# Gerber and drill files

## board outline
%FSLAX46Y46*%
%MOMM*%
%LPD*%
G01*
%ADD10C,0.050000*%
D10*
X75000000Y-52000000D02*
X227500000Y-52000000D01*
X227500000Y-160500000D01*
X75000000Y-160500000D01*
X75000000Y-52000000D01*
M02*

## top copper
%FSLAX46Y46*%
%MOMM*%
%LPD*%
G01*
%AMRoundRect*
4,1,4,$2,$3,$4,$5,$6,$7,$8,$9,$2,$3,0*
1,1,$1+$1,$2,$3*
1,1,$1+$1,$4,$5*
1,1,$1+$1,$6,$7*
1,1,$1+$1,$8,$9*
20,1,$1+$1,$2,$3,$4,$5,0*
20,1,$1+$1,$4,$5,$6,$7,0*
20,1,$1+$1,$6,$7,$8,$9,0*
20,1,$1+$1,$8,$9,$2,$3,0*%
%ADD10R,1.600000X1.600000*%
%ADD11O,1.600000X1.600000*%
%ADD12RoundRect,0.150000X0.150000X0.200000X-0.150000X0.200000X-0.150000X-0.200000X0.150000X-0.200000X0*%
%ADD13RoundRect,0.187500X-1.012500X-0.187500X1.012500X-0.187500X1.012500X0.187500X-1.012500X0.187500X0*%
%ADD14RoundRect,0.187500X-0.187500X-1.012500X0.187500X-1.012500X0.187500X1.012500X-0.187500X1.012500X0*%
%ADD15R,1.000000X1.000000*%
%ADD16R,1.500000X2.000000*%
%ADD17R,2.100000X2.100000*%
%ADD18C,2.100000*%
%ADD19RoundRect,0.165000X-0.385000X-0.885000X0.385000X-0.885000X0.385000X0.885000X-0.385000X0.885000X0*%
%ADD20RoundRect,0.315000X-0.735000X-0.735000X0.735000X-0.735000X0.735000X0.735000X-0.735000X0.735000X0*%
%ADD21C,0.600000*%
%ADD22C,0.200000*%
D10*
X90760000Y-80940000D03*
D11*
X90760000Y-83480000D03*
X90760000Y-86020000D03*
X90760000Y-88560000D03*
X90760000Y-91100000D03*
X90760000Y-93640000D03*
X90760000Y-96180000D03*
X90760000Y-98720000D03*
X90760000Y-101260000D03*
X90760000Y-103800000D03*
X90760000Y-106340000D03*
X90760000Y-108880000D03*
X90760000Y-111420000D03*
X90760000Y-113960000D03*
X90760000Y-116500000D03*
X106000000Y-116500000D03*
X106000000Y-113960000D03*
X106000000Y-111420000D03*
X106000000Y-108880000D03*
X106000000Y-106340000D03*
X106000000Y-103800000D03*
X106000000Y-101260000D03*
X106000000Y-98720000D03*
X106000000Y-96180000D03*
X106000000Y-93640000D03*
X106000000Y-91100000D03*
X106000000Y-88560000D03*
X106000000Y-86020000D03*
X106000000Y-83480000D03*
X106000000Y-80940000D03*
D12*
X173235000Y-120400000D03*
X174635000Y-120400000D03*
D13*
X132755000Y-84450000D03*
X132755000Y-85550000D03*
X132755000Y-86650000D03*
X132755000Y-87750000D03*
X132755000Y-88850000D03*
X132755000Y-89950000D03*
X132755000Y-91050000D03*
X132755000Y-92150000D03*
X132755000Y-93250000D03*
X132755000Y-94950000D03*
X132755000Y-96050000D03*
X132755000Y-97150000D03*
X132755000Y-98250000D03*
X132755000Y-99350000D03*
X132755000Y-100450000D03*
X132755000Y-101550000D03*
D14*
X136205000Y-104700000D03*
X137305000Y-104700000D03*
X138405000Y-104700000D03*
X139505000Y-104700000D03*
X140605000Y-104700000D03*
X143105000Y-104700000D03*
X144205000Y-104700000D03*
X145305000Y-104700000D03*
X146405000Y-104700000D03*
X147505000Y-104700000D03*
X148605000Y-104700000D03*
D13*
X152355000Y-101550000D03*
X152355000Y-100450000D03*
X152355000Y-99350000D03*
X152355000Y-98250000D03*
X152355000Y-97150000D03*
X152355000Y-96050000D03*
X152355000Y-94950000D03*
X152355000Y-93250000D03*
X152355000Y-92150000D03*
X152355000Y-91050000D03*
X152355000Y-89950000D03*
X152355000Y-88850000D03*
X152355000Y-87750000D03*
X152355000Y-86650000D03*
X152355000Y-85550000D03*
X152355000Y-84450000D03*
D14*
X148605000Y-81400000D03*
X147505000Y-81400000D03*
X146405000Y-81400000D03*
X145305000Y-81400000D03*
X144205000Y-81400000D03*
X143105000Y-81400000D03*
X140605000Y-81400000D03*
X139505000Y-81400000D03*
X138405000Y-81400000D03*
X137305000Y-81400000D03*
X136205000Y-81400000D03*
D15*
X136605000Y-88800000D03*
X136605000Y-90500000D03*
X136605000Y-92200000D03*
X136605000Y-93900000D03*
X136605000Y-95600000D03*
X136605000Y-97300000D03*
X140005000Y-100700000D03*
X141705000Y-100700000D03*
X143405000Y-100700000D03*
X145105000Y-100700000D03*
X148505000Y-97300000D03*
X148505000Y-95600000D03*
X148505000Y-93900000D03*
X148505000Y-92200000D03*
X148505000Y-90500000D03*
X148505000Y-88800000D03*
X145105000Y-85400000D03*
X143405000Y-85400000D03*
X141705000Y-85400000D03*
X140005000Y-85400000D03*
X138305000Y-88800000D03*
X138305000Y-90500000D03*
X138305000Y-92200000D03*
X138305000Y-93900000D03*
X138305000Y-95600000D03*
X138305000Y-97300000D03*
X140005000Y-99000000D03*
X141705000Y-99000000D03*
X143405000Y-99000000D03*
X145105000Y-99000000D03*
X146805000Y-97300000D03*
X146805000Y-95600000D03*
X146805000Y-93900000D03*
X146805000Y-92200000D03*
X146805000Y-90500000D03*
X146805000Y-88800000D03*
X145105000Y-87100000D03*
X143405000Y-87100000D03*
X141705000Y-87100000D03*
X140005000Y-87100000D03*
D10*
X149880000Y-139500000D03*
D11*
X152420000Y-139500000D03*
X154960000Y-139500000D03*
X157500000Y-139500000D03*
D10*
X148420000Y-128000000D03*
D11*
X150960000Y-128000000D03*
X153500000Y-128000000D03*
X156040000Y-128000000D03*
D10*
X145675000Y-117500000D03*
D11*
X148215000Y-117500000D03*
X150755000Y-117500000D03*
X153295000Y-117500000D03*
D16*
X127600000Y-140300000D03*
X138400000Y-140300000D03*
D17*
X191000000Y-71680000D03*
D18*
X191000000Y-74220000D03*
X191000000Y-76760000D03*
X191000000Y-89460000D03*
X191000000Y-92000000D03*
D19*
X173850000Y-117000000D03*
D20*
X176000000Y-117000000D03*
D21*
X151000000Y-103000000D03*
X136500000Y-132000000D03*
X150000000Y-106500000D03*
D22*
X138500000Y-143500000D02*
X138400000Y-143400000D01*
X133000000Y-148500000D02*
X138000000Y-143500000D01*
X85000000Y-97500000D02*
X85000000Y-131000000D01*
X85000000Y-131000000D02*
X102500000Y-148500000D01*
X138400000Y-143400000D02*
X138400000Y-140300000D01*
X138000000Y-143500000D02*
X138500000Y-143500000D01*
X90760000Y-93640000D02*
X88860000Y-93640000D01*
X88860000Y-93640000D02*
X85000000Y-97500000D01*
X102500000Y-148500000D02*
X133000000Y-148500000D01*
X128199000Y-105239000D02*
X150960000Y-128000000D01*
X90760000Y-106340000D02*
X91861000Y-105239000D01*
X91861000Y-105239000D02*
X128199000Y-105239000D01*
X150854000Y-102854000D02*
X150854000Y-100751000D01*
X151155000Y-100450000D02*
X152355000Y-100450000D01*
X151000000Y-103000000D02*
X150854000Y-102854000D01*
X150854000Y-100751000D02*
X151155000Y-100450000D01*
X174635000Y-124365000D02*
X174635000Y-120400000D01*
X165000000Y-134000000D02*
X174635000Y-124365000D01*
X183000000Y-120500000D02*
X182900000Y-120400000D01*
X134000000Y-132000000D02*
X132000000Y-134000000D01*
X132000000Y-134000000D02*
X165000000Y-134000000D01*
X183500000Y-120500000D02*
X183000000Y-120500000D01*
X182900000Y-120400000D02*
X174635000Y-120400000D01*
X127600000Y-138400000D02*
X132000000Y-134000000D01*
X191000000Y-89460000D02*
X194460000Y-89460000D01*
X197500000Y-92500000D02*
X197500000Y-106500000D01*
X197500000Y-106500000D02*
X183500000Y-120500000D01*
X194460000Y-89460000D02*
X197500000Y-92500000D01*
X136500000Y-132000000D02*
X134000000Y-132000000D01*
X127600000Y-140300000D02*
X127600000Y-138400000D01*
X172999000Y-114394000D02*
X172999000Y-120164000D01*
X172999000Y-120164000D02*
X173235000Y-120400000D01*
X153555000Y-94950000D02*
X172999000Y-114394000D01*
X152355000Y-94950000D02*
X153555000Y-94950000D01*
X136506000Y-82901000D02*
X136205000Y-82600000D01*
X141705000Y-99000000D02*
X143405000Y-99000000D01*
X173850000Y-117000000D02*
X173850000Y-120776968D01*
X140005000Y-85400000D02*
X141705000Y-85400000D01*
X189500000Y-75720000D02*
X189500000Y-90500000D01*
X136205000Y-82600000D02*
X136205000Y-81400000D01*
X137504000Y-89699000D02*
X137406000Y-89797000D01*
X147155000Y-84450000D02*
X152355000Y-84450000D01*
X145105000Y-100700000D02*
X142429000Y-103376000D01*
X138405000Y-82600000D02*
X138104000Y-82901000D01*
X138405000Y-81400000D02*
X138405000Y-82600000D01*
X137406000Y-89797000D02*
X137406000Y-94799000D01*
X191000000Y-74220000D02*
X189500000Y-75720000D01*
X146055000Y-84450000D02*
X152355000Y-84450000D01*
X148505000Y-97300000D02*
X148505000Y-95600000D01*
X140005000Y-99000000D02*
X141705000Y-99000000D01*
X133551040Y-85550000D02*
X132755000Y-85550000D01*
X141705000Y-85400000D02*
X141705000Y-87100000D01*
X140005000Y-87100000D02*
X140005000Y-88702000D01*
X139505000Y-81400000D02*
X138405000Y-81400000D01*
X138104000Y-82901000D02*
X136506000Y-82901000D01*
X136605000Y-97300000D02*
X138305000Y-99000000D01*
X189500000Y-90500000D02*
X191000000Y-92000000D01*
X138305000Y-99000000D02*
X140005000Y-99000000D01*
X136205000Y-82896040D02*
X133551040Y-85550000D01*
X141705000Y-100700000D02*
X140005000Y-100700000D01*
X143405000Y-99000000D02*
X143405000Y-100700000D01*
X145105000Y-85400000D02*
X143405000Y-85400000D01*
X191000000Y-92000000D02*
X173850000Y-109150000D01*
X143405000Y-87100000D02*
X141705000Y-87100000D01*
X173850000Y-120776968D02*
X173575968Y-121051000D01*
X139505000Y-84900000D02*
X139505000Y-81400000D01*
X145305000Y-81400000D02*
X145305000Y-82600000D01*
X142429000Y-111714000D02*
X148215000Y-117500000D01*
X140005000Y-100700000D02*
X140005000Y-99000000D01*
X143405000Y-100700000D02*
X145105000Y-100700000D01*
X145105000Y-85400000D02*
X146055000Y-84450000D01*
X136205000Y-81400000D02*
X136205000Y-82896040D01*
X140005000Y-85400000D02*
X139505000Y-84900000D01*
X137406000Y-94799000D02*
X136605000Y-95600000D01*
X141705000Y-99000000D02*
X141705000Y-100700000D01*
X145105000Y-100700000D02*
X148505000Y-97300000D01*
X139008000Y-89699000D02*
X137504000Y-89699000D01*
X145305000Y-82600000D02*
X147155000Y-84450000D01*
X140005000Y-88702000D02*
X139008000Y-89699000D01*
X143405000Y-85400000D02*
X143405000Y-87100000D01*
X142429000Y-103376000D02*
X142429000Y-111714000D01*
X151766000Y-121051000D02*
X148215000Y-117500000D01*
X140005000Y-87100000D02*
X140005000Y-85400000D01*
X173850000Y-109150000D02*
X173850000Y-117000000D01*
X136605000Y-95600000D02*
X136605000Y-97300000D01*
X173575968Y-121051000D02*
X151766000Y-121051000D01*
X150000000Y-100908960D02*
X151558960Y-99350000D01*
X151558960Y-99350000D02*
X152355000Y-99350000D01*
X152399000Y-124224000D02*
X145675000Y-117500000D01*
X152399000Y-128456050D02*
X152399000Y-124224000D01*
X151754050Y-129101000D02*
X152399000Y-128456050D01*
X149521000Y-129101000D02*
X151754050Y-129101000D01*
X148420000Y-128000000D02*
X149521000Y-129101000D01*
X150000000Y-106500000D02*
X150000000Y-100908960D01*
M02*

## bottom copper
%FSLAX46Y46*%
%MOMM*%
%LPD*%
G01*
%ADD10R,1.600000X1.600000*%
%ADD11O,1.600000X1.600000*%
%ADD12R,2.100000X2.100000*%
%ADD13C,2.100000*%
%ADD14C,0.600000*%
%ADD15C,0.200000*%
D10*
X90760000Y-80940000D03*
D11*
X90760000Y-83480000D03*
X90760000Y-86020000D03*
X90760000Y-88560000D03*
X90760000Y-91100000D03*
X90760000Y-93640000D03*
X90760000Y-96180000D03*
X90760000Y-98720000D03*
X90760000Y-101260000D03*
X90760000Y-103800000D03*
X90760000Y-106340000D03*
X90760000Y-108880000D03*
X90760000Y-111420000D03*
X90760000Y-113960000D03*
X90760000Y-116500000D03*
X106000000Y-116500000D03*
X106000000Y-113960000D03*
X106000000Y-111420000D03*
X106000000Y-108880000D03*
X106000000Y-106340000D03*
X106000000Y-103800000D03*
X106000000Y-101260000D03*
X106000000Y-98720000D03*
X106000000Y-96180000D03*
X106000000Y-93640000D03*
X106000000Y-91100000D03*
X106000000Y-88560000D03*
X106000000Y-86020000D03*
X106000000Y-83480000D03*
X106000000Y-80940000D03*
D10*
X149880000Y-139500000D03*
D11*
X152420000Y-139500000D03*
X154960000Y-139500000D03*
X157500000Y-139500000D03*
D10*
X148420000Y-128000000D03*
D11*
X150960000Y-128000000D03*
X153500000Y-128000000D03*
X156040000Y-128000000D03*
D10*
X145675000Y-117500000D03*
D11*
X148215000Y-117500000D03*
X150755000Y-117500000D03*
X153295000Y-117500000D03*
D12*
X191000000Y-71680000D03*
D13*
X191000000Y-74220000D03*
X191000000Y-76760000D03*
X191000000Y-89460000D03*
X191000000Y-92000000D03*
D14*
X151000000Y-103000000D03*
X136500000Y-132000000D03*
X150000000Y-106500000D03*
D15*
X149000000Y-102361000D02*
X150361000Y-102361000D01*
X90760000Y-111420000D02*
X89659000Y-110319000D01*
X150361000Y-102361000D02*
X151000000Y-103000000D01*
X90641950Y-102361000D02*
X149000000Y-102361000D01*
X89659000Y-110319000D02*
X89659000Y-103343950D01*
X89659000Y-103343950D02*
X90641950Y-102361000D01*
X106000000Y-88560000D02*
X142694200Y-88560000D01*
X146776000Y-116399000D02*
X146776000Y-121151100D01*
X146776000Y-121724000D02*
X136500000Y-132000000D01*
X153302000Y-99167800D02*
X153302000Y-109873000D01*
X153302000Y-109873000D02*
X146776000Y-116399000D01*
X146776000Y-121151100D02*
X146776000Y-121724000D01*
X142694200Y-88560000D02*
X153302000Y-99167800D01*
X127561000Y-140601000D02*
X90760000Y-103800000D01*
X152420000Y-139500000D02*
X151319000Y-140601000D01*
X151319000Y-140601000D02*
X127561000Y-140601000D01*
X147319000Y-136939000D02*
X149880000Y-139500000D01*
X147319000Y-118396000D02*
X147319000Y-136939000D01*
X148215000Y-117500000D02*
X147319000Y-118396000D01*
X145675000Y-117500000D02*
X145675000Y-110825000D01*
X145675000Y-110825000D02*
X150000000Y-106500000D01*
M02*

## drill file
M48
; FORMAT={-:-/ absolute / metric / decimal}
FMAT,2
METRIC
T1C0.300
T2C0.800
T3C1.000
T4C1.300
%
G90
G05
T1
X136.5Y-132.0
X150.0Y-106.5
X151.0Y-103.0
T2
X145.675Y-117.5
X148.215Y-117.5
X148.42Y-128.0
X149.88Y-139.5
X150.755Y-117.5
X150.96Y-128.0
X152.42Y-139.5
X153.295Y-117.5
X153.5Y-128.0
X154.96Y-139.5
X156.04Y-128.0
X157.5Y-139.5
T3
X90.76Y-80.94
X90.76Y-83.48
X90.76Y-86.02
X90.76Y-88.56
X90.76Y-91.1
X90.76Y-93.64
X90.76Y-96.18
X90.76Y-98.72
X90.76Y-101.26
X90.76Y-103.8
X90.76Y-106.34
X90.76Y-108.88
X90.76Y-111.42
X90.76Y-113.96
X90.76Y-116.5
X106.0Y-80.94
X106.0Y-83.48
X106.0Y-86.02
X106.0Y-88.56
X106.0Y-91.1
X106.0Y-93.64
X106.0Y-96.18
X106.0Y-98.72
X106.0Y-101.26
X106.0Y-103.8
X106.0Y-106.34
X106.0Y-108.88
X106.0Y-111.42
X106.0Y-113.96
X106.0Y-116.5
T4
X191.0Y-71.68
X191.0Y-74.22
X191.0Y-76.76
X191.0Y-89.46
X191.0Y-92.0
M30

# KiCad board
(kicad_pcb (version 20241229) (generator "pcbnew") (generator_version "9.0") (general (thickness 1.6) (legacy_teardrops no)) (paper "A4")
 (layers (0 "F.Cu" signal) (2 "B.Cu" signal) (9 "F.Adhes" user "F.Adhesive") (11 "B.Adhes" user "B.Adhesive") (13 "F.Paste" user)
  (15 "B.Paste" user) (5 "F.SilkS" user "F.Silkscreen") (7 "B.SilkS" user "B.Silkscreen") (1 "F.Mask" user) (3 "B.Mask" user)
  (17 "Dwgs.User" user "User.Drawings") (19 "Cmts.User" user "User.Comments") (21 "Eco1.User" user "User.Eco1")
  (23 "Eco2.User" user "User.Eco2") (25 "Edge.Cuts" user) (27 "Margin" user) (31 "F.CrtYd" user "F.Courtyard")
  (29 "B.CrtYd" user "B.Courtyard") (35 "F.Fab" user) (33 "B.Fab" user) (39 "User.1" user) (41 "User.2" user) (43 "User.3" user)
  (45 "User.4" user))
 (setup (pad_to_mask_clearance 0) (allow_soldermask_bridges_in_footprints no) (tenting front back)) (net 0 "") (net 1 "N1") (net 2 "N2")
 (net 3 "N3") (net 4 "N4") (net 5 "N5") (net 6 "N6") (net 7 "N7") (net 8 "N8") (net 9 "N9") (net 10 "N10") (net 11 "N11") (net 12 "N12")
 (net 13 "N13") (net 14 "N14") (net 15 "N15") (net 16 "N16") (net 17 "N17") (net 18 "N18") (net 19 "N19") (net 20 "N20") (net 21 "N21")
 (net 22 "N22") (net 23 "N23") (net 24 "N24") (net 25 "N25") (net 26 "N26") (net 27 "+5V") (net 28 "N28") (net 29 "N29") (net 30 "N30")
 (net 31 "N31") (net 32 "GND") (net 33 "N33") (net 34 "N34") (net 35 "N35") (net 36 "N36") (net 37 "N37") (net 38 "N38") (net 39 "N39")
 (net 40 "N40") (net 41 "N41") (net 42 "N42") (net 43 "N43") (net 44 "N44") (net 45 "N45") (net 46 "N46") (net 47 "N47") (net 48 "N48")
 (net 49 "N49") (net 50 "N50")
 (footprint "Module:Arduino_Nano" (layer "F.Cu") (at 90.76 80.94)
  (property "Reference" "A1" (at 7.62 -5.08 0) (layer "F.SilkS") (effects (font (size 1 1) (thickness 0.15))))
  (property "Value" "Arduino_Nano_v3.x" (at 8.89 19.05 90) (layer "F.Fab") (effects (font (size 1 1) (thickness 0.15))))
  (pad "1" thru_hole rect (at 0 0) (size 1.6 1.6) (drill 1) (layers "*.Cu" "*.Mask") (remove_unused_layers no) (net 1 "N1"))
  (pad "2" thru_hole oval (at 0 2.54) (size 1.6 1.6) (drill 1) (layers "*.Cu" "*.Mask") (remove_unused_layers no) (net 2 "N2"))
  (pad "3" thru_hole oval (at 0 5.08) (size 1.6 1.6) (drill 1) (layers "*.Cu" "*.Mask") (remove_unused_layers no) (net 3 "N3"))
  (pad "4" thru_hole oval (at 0 7.62) (size 1.6 1.6) (drill 1) (layers "*.Cu" "*.Mask") (remove_unused_layers no) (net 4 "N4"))
  (pad "5" thru_hole oval (at 0 10.16) (size 1.6 1.6) (drill 1) (layers "*.Cu" "*.Mask") (remove_unused_layers no) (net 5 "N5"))
  (pad "6" thru_hole oval (at 0 12.7) (size 1.6 1.6) (drill 1) (layers "*.Cu" "*.Mask") (remove_unused_layers no) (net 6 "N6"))
  (pad "7" thru_hole oval (at 0 15.24) (size 1.6 1.6) (drill 1) (layers "*.Cu" "*.Mask") (remove_unused_layers no) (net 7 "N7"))
  (pad "8" thru_hole oval (at 0 17.78) (size 1.6 1.6) (drill 1) (layers "*.Cu" "*.Mask") (remove_unused_layers no) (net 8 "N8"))
  (pad "9" thru_hole oval (at 0 20.32) (size 1.6 1.6) (drill 1) (layers "*.Cu" "*.Mask") (remove_unused_layers no) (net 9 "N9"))
  (pad "10" thru_hole oval (at 0 22.86) (size 1.6 1.6) (drill 1) (layers "*.Cu" "*.Mask") (remove_unused_layers no) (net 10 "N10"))
  (pad "11" thru_hole oval (at 0 25.4) (size 1.6 1.6) (drill 1) (layers "*.Cu" "*.Mask") (remove_unused_layers no) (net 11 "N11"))
  (pad "12" thru_hole oval (at 0 27.94) (size 1.6 1.6) (drill 1) (layers "*.Cu" "*.Mask") (remove_unused_layers no) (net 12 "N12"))
  (pad "13" thru_hole oval (at 0 30.48) (size 1.6 1.6) (drill 1) (layers "*.Cu" "*.Mask") (remove_unused_layers no) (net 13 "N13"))
  (pad "14" thru_hole oval (at 0 33.02) (size 1.6 1.6) (drill 1) (layers "*.Cu" "*.Mask") (remove_unused_layers no) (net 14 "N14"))
  (pad "15" thru_hole oval (at 0 35.56) (size 1.6 1.6) (drill 1) (layers "*.Cu" "*.Mask") (remove_unused_layers no) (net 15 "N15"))
  (pad "16" thru_hole oval (at 15.24 35.56) (size 1.6 1.6) (drill 1) (layers "*.Cu" "*.Mask") (remove_unused_layers no) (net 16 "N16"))
  (pad "17" thru_hole oval (at 15.24 33.02) (size 1.6 1.6) (drill 1) (layers "*.Cu" "*.Mask") (remove_unused_layers no) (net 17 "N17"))
  (pad "18" thru_hole oval (at 15.24 30.48) (size 1.6 1.6) (drill 1) (layers "*.Cu" "*.Mask") (remove_unused_layers no) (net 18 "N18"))
  (pad "19" thru_hole oval (at 15.24 27.94) (size 1.6 1.6) (drill 1) (layers "*.Cu" "*.Mask") (remove_unused_layers no) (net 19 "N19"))
  (pad "20" thru_hole oval (at 15.24 25.4) (size 1.6 1.6) (drill 1) (layers "*.Cu" "*.Mask") (remove_unused_layers no) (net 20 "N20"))
  (pad "21" thru_hole oval (at 15.24 22.86) (size 1.6 1.6) (drill 1) (layers "*.Cu" "*.Mask") (remove_unused_layers no) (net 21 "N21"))
  (pad "22" thru_hole oval (at 15.24 20.32) (size 1.6 1.6) (drill 1) (layers "*.Cu" "*.Mask") (remove_unused_layers no) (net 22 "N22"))
  (pad "23" thru_hole oval (at 15.24 17.78) (size 1.6 1.6) (drill 1) (layers "*.Cu" "*.Mask") (remove_unused_layers no) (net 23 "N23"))
  (pad "24" thru_hole oval (at 15.24 15.24) (size 1.6 1.6) (drill 1) (layers "*.Cu" "*.Mask") (remove_unused_layers no) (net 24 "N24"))
  (pad "25" thru_hole oval (at 15.24 12.7) (size 1.6 1.6) (drill 1) (layers "*.Cu" "*.Mask") (remove_unused_layers no) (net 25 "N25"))
  (pad "26" thru_hole oval (at 15.24 10.16) (size 1.6 1.6) (drill 1) (layers "*.Cu" "*.Mask") (remove_unused_layers no) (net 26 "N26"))
  (pad "27" thru_hole oval (at 15.24 7.62) (size 1.6 1.6) (drill 1) (layers "*.Cu" "*.Mask") (remove_unused_layers no) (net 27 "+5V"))
  (pad "28" thru_hole oval (at 15.24 5.08) (size 1.6 1.6) (drill 1) (layers "*.Cu" "*.Mask") (remove_unused_layers no) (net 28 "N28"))
  (pad "29" thru_hole oval (at 15.24 2.54) (size 1.6 1.6) (drill 1) (layers "*.Cu" "*.Mask") (remove_unused_layers no) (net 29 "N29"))
  (pad "30" thru_hole oval (at 15.24 0) (size 1.6 1.6) (drill 1) (layers "*.Cu" "*.Mask") (remove_unused_layers no) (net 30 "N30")))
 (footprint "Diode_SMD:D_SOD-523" (layer "F.Cu") (at 173.935 120.4)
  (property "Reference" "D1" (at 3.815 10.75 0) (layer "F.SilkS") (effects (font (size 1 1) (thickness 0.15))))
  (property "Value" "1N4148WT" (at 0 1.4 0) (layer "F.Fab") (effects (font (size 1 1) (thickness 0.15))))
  (pad "1" smd roundrect (at -0.7 0 180) (size 0.6 0.7) (layers "F.Cu" "F.Mask" "F.Paste") (roundrect_rratio 0.25) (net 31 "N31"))
  (pad "2" smd roundrect (at 0.7 0 180) (size 0.6 0.7) (layers "F.Cu" "F.Mask" "F.Paste") (roundrect_rratio 0.25) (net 27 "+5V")))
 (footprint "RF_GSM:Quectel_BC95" (layer "F.Cu") (at 142.555 93.05)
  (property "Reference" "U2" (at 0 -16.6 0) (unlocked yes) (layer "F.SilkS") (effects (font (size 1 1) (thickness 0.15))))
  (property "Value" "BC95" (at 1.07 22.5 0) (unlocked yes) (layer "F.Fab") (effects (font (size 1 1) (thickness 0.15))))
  (pad "" smd roundrect (at -10.1 -8.6) (size 2.6 0.6375) (layers "F.Paste") (roundrect_rratio 0.25))
  (pad "" smd roundrect (at -10.1 -7.5) (size 2.6 0.6375) (layers "F.Paste") (roundrect_rratio 0.25))
  (pad "" smd roundrect (at -10.1 -6.4) (size 2.6 0.6375) (layers "F.Paste") (roundrect_rratio 0.25))
  (pad "" smd roundrect (at -10.1 -5.3) (size 2.6 0.6375) (layers "F.Paste") (roundrect_rratio 0.25))
  (pad "" smd roundrect (at -10.1 -4.2) (size 2.6 0.6375) (layers "F.Paste") (roundrect_rratio 0.25))
  (pad "" smd roundrect (at -10.1 -3.1) (size 2.6 0.6375) (layers "F.Paste") (roundrect_rratio 0.25))
  (pad "" smd roundrect (at -10.1 -2) (size 2.6 0.6375) (layers "F.Paste") (roundrect_rratio 0.25))
  (pad "" smd roundrect (at -10.1 -0.9) (size 2.6 0.6375) (layers "F.Paste") (roundrect_rratio 0.25))
  (pad "" smd roundrect (at -10.1 0.2) (size 2.6 0.6375) (layers "F.Paste") (roundrect_rratio 0.25))
  (pad "" smd roundrect (at -10.1 1.9) (size 2.6 0.6375) (layers "F.Paste") (roundrect_rratio 0.25))
  (pad "" smd roundrect (at -10.1 3) (size 2.6 0.6375) (layers "F.Paste") (roundrect_rratio 0.25))
  (pad "" smd roundrect (at -10.1 4.1) (size 2.6 0.6375) (layers "F.Paste") (roundrect_rratio 0.25))
  (pad "" smd roundrect (at -10.1 5.2) (size 2.6 0.6375) (layers "F.Paste") (roundrect_rratio 0.25))
  (pad "" smd roundrect (at -10.1 6.3) (size 2.6 0.6375) (layers "F.Paste") (roundrect_rratio 0.25))
  (pad "" smd roundrect (at -10.1 7.4) (size 2.6 0.6375) (layers "F.Paste") (roundrect_rratio 0.25))
  (pad "" smd roundrect (at -10.1 8.5) (size 2.6 0.6375) (layers "F.Paste") (roundrect_rratio 0.25))
  (pad "" smd roundrect (at -6.35 -11.95 90) (size 2.6 0.6375) (layers "F.Paste") (roundrect_rratio 0.25))
  (pad "" smd roundrect (at -6.35 11.95 90) (size 2.6 0.6375) (layers "F.Paste") (roundrect_rratio 0.25))
  (pad "" smd circle (at -5.95 -4.25) (size 0.9 0.9) (layers "F.Paste"))
  (pad "" smd circle (at -5.95 -2.55) (size 0.9 0.9) (layers "F.Paste"))
  (pad "" smd circle (at -5.95 -0.85) (size 0.9 0.9) (layers "F.Paste"))
  (pad "" smd circle (at -5.95 0.85) (size 0.9 0.9) (layers "F.Paste"))
  (pad "" smd circle (at -5.95 2.55) (size 0.9 0.9) (layers "F.Paste"))
  (pad "" smd circle (at -5.95 4.25) (size 0.9 0.9) (layers "F.Paste"))
  (pad "" smd roundrect (at -5.25 -11.95 90) (size 2.6 0.6375) (layers "F.Paste") (roundrect_rratio 0.25))
  (pad "" smd roundrect (at -5.25 11.95 90) (size 2.6 0.6375) (layers "F.Paste") (roundrect_rratio 0.25))
  (pad "" smd circle (at -4.25 -4.25) (size 0.9 0.9) (layers "F.Paste"))
  (pad "" smd circle (at -4.25 -2.55) (size 0.9 0.9) (layers "F.Paste"))
  (pad "" smd circle (at -4.25 -0.85) (size 0.9 0.9) (layers "F.Paste"))
  (pad "" smd circle (at -4.25 0.85) (size 0.9 0.9) (layers "F.Paste"))
  (pad "" smd circle (at -4.25 2.55) (size 0.9 0.9) (layers "F.Paste"))
  (pad "" smd circle (at -4.25 4.25) (size 0.9 0.9) (layers "F.Paste"))
  (pad "" smd roundrect (at -4.15 -11.95 90) (size 2.6 0.6375) (layers "F.Paste") (roundrect_rratio 0.25))
  (pad "" smd roundrect (at -4.15 11.95 90) (size 2.6 0.6375) (layers "F.Paste") (roundrect_rratio 0.25))
  (pad "" smd roundrect (at -3.05 -11.95 90) (size 2.6 0.6375) (layers "F.Paste") (roundrect_rratio 0.25))
  (pad "" smd roundrect (at -3.05 11.95 90) (size 2.6 0.6375) (layers "F.Paste") (roundrect_rratio 0.25))
  (pad "" smd circle (at -2.55 -7.65) (size 0.9 0.9) (layers "F.Paste"))
  (pad "" smd circle (at -2.55 -5.95) (size 0.9 0.9) (layers "F.Paste"))
  (pad "" smd circle (at -2.55 5.95) (size 0.9 0.9) (layers "F.Paste"))
  (pad "" smd circle (at -2.55 7.65) (size 0.9 0.9) (layers "F.Paste"))
  (pad "" smd roundrect (at -1.95 -11.95 90) (size 2.6 0.6375) (layers "F.Paste") (roundrect_rratio 0.25))
  (pad "" smd roundrect (at -1.95 11.95 90) (size 2.6 0.6375) (layers "F.Paste") (roundrect_rratio 0.25))
  (pad "" smd circle (at -0.85 -7.65) (size 0.9 0.9) (layers "F.Paste"))
  (pad "" smd circle (at -0.85 -5.95) (size 0.9 0.9) (layers "F.Paste"))
  (pad "" smd circle (at -0.85 5.95) (size 0.9 0.9) (layers "F.Paste"))
  (pad "" smd circle (at -0.85 7.65) (size 0.9 0.9) (layers "F.Paste"))
  (pad "" smd roundrect (at 0.55 -11.95 90) (size 2.6 0.6375) (layers "F.Paste") (roundrect_rratio 0.25))
  (pad "" smd roundrect (at 0.55 11.95 90) (size 2.6 0.6375) (layers "F.Paste") (roundrect_rratio 0.25))
  (pad "" smd circle (at 0.85 -7.65) (size 0.9 0.9) (layers "F.Paste"))
  (pad "" smd circle (at 0.85 -5.95) (size 0.9 0.9) (layers "F.Paste"))
  (pad "" smd circle (at 0.85 5.95) (size 0.9 0.9) (layers "F.Paste"))
  (pad "" smd circle (at 0.85 7.65) (size 0.9 0.9) (layers "F.Paste"))
  (pad "" smd roundrect (at 1.65 -11.95 90) (size 2.6 0.6375) (layers "F.Paste") (roundrect_rratio 0.25))
  (pad "" smd roundrect (at 1.65 11.95 90) (size 2.6 0.6375) (layers "F.Paste") (roundrect_rratio 0.25))
  (pad "" smd circle (at 2.55 -7.65) (size 0.9 0.9) (layers "F.Paste"))
  (pad "" smd circle (at 2.55 -5.95) (size 0.9 0.9) (layers "F.Paste"))
  (pad "" smd circle (at 2.55 5.95) (size 0.9 0.9) (layers "F.Paste"))
  (pad "" smd circle (at 2.55 7.65) (size 0.9 0.9) (layers "F.Paste"))
  (pad "" smd roundrect (at 2.75 -11.95 90) (size 2.6 0.6375) (layers "F.Paste") (roundrect_rratio 0.25))
  (pad "" smd roundrect (at 2.75 11.95 90) (size 2.6 0.6375) (layers "F.Paste") (roundrect_rratio 0.25))
  (pad "" smd roundrect (at 3.85 -11.95 90) (size 2.6 0.6375) (layers "F.Paste") (roundrect_rratio 0.25))
  (pad "" smd roundrect (at 3.85 11.95 90) (size 2.6 0.6375) (layers "F.Paste") (roundrect_rratio 0.25))
  (pad "" smd circle (at 4.25 -4.25) (size 0.9 0.9) (layers "F.Paste"))
  (pad "" smd circle (at 4.25 -2.55) (size 0.9 0.9) (layers "F.Paste"))
  (pad "" smd circle (at 4.25 -0.85) (size 0.9 0.9) (layers "F.Paste"))
  (pad "" smd circle (at 4.25 0.85) (size 0.9 0.9) (layers "F.Paste"))
  (pad "" smd circle (at 4.25 2.55) (size 0.9 0.9) (layers "F.Paste"))
  (pad "" smd circle (at 4.25 4.25) (size 0.9 0.9) (layers "F.Paste"))
  (pad "" smd roundrect (at 4.95 -11.95 90) (size 2.6 0.6375) (layers "F.Paste") (roundrect_rratio 0.25))
  (pad "" smd roundrect (at 4.95 11.95 90) (size 2.6 0.6375) (layers "F.Paste") (roundrect_rratio 0.25))
  (pad "" smd circle (at 5.95 -4.25) (size 0.9 0.9) (layers "F.Paste"))
  (pad "" smd circle (at 5.95 -2.55) (size 0.9 0.9) (layers "F.Paste"))
  (pad "" smd circle (at 5.95 -0.85) (size 0.9 0.9) (layers "F.Paste"))
  (pad "" smd circle (at 5.95 0.85) (size 0.9 0.9) (layers "F.Paste"))
  (pad "" smd circle (at 5.95 2.55) (size 0.9 0.9) (layers "F.Paste"))
  (pad "" smd circle (at 5.95 4.25) (size 0.9 0.9) (layers "F.Paste"))
  (pad "" smd roundrect (at 6.05 -11.95 90) (size 2.6 0.6375) (layers "F.Paste") (roundrect_rratio 0.25))
  (pad "" smd roundrect (at 6.05 11.95 90) (size 2.6 0.6375) (layers "F.Paste") (roundrect_rratio 0.25))
  (pad "" smd roundrect (at 10.1 -8.6) (size 2.6 0.6375) (layers "F.Paste") (roundrect_rratio 0.25))
  (pad "" smd roundrect (at 10.1 -7.5) (size 2.6 0.6375) (layers "F.Paste") (roundrect_rratio 0.25))
  (pad "" smd roundrect (at 10.1 -6.4) (size 2.6 0.6375) (layers "F.Paste") (roundrect_rratio 0.25))
  (pad "" smd roundrect (at 10.1 -5.3) (size 2.6 0.6375) (layers "F.Paste") (roundrect_rratio 0.25))
  (pad "" smd roundrect (at 10.1 -4.2) (size 2.6 0.6375) (layers "F.Paste") (roundrect_rratio 0.25))
  (pad "" smd roundrect (at 10.1 -3.1) (size 2.6 0.6375) (layers "F.Paste") (roundrect_rratio 0.25))
  (pad "" smd roundrect (at 10.1 -2) (size 2.6 0.6375) (layers "F.Paste") (roundrect_rratio 0.25))
  (pad "" smd roundrect (at 10.1 -0.9) (size 2.6 0.6375) (layers "F.Paste") (roundrect_rratio 0.25))
  (pad "" smd roundrect (at 10.1 0.2) (size 2.6 0.6375) (layers "F.Paste") (roundrect_rratio 0.25))
  (pad "" smd roundrect (at 10.1 1.9) (size 2.6 0.6375) (layers "F.Paste") (roundrect_rratio 0.25))
  (pad "" smd roundrect (at 10.1 3) (size 2.6 0.6375) (layers "F.Paste") (roundrect_rratio 0.25))
  (pad "" smd roundrect (at 10.1 4.1) (size 2.6 0.6375) (layers "F.Paste") (roundrect_rratio 0.25))
  (pad "" smd roundrect (at 10.1 5.2) (size 2.6 0.6375) (layers "F.Paste") (roundrect_rratio 0.25))
  (pad "" smd roundrect (at 10.1 6.3) (size 2.6 0.6375) (layers "F.Paste") (roundrect_rratio 0.25))
  (pad "" smd roundrect (at 10.1 7.4) (size 2.6 0.6375) (layers "F.Paste") (roundrect_rratio 0.25))
  (pad "" smd roundrect (at 10.1 8.5) (size 2.6 0.6375) (layers "F.Paste") (roundrect_rratio 0.25))
  (pad "1" smd roundrect (at -9.8 -8.6) (size 2.4 0.75) (layers "F.Cu" "F.Mask") (roundrect_rratio 0.25))
  (pad "2" smd roundrect (at -9.8 -7.5) (size 2.4 0.75) (layers "F.Cu" "F.Mask") (roundrect_rratio 0.25) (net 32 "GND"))
  (pad "3" smd roundrect (at -9.8 -6.4) (size 2.4 0.75) (layers "F.Cu" "F.Mask") (roundrect_rratio 0.25))
  (pad "4" smd roundrect (at -9.8 -5.3) (size 2.4 0.75) (layers "F.Cu" "F.Mask") (roundrect_rratio 0.25))
  (pad "5" smd roundrect (at -9.8 -4.2) (size 2.4 0.75) (layers "F.Cu" "F.Mask") (roundrect_rratio 0.25))
  (pad "6" smd roundrect (at -9.8 -3.1) (size 2.4 0.75) (layers "F.Cu" "F.Mask") (roundrect_rratio 0.25))
  (pad "7" smd roundrect (at -9.8 -2) (size 2.4 0.75) (layers "F.Cu" "F.Mask") (roundrect_rratio 0.25))
  (pad "8" smd roundrect (at -9.8 -0.9) (size 2.4 0.75) (layers "F.Cu" "F.Mask") (roundrect_rratio 0.25))
  (pad "9" smd roundrect (at -9.8 0.2) (size 2.4 0.75) (layers "F.Cu" "F.Mask") (roundrect_rratio 0.25))
  (pad "10" smd roundrect (at -9.8 1.9) (size 2.4 0.75) (layers "F.Cu" "F.Mask") (roundrect_rratio 0.25))
  (pad "11" smd roundrect (at -9.8 3) (size 2.4 0.75) (layers "F.Cu" "F.Mask") (roundrect_rratio 0.25))
  (pad "12" smd roundrect (at -9.8 4.1) (size 2.4 0.75) (layers "F.Cu" "F.Mask") (roundrect_rratio 0.25))
  (pad "13" smd roundrect (at -9.8 5.2) (size 2.4 0.75) (layers "F.Cu" "F.Mask") (roundrect_rratio 0.25))
  (pad "14" smd roundrect (at -9.8 6.3) (size 2.4 0.75) (layers "F.Cu" "F.Mask") (roundrect_rratio 0.25))
  (pad "15" smd roundrect (at -9.8 7.4) (size 2.4 0.75) (layers "F.Cu" "F.Mask") (roundrect_rratio 0.25) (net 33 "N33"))
  (pad "16" smd roundrect (at -9.8 8.5) (size 2.4 0.75) (layers "F.Cu" "F.Mask") (roundrect_rratio 0.25))
  (pad "17" smd roundrect (at -6.35 11.65) (size 0.75 2.4) (layers "F.Cu" "F.Mask") (roundrect_rratio 0.25))
  (pad "18" smd roundrect (at -5.25 11.65) (size 0.75 2.4) (layers "F.Cu" "F.Mask") (roundrect_rratio 0.25) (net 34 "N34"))
  (pad "19" smd roundrect (at -4.15 11.65) (size 0.75 2.4) (layers "F.Cu" "F.Mask") (roundrect_rratio 0.25) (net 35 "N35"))
  (pad "20" smd roundrect (at -3.05 11.65) (size 0.75 2.4) (layers "F.Cu" "F.Mask") (roundrect_rratio 0.25) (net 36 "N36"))
  (pad "21" smd roundrect (at -1.95 11.65) (size 0.75 2.4) (layers "F.Cu" "F.Mask") (roundrect_rratio 0.25) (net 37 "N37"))
  (pad "22" smd roundrect (at 0.55 11.65) (size 0.75 2.4) (layers "F.Cu" "F.Mask") (roundrect_rratio 0.25))
  (pad "23" smd roundrect (at 1.65 11.65) (size 0.75 2.4) (layers "F.Cu" "F.Mask") (roundrect_rratio 0.25))
  (pad "24" smd roundrect (at 2.75 11.65) (size 0.75 2.4) (layers "F.Cu" "F.Mask") (roundrect_rratio 0.25))
  (pad "25" smd roundrect (at 3.85 11.65) (size 0.75 2.4) (layers "F.Cu" "F.Mask") (roundrect_rratio 0.25))
  (pad "26" smd roundrect (at 4.95 11.65) (size 0.75 2.4) (layers "F.Cu" "F.Mask") (roundrect_rratio 0.25) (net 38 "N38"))
  (pad "27" smd roundrect (at 6.05 11.65) (size 0.75 2.4) (layers "F.Cu" "F.Mask") (roundrect_rratio 0.25))
  (pad "28" smd roundrect (at 9.8 8.5) (size 2.4 0.75) (layers "F.Cu" "F.Mask") (roundrect_rratio 0.25))
  (pad "29" smd roundrect (at 9.8 7.4) (size 2.4 0.75) (layers "F.Cu" "F.Mask") (roundrect_rratio 0.25) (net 13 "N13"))
  (pad "30" smd roundrect (at 9.8 6.3) (size 2.4 0.75) (layers "F.Cu" "F.Mask") (roundrect_rratio 0.25) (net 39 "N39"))
  (pad "31" smd roundrect (at 9.8 5.2) (size 2.4 0.75) (layers "F.Cu" "F.Mask") (roundrect_rratio 0.25))
  (pad "32" smd roundrect (at 9.8 4.1) (size 2.4 0.75) (layers "F.Cu" "F.Mask") (roundrect_rratio 0.25))
  (pad "33" smd roundrect (at 9.8 3) (size 2.4 0.75) (layers "F.Cu" "F.Mask") (roundrect_rratio 0.25))
  (pad "34" smd roundrect (at 9.8 1.9) (size 2.4 0.75) (layers "F.Cu" "F.Mask") (roundrect_rratio 0.25) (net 31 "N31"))
  (pad "35" smd roundrect (at 9.8 0.2) (size 2.4 0.75) (layers "F.Cu" "F.Mask") (roundrect_rratio 0.25))
  (pad "36" smd roundrect (at 9.8 -0.9) (size 2.4 0.75) (layers "F.Cu" "F.Mask") (roundrect_rratio 0.25))
  (pad "37" smd roundrect (at 9.8 -2) (size 2.4 0.75) (layers "F.Cu" "F.Mask") (roundrect_rratio 0.25))
  (pad "38" smd roundrect (at 9.8 -3.1) (size 2.4 0.75) (layers "F.Cu" "F.Mask") (roundrect_rratio 0.25) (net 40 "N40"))
  (pad "39" smd roundrect (at 9.8 -4.2) (size 2.4 0.75) (layers "F.Cu" "F.Mask") (roundrect_rratio 0.25) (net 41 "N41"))
  (pad "40" smd roundrect (at 9.8 -5.3) (size 2.4 0.75) (layers "F.Cu" "F.Mask") (roundrect_rratio 0.25) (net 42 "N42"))
  (pad "41" smd roundrect (at 9.8 -6.4) (size 2.4 0.75) (layers "F.Cu" "F.Mask") (roundrect_rratio 0.25) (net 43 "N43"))
  (pad "42" smd roundrect (at 9.8 -7.5) (size 2.4 0.75) (layers "F.Cu" "F.Mask") (roundrect_rratio 0.25) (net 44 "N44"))
  (pad "43" smd roundrect (at 9.8 -8.6) (size 2.4 0.75) (layers "F.Cu" "F.Mask") (roundrect_rratio 0.25) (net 32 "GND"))
  (pad "44" smd roundrect (at 6.05 -11.65) (size 0.75 2.4) (layers "F.Cu" "F.Mask") (roundrect_rratio 0.25))
  (pad "45" smd roundrect (at 4.95 -11.65) (size 0.75 2.4) (layers "F.Cu" "F.Mask") (roundrect_rratio 0.25) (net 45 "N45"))
  (pad "46" smd roundrect (at 3.85 -11.65) (size 0.75 2.4) (layers "F.Cu" "F.Mask") (roundrect_rratio 0.25) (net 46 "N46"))
  (pad "47" smd roundrect (at 2.75 -11.65) (size 0.75 2.4) (layers "F.Cu" "F.Mask") (roundrect_rratio 0.25) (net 32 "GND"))
  (pad "48" smd roundrect (at 1.65 -11.65) (size 0.75 2.4) (layers "F.Cu" "F.Mask") (roundrect_rratio 0.25) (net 32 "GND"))
  (pad "49" smd roundrect (at 0.55 -11.65) (size 0.75 2.4) (layers "F.Cu" "F.Mask") (roundrect_rratio 0.25))
  (pad "50" smd roundrect (at -1.95 -11.65) (size 0.75 2.4) (layers "F.Cu" "F.Mask") (roundrect_rratio 0.25))
  (pad "51" smd roundrect (at -3.05 -11.65) (size 0.75 2.4) (layers "F.Cu" "F.Mask") (roundrect_rratio 0.25) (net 32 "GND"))
  (pad "52" smd roundrect (at -4.15 -11.65) (size 0.75 2.4) (layers "F.Cu" "F.Mask") (roundrect_rratio 0.25) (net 32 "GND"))
  (pad "53" smd roundrect (at -5.25 -11.65) (size 0.75 2.4) (layers "F.Cu" "F.Mask") (roundrect_rratio 0.25) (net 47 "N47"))
  (pad "54" smd roundrect (at -6.35 -11.65) (size 0.75 2.4) (layers "F.Cu" "F.Mask") (roundrect_rratio 0.25) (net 32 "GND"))
  (pad "55" smd rect (at -5.95 -4.25) (size 1 1) (layers "F.Cu" "F.Mask"))
  (pad "56" smd rect (at -5.95 -2.55) (size 1 1) (layers "F.Cu" "F.Mask"))
  (pad "57" smd rect (at -5.95 -0.85) (size 1 1) (layers "F.Cu" "F.Mask"))
  (pad "58" smd rect (at -5.95 0.85) (size 1 1) (layers "F.Cu" "F.Mask"))
  (pad "59" smd rect (at -5.95 2.55) (size 1 1) (layers "F.Cu" "F.Mask") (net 32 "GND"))
  (pad "60" smd rect (at -5.95 4.25) (size 1 1) (layers "F.Cu" "F.Mask") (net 32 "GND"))
  (pad "61" smd rect (at -2.55 7.65) (size 1 1) (layers "F.Cu" "F.Mask") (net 32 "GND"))
  (pad "62" smd rect (at -0.85 7.65) (size 1 1) (layers "F.Cu" "F.Mask") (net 32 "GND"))
  (pad "63" smd rect (at 0.85 7.65) (size 1 1) (layers "F.Cu" "F.Mask") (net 32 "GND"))
  (pad "64" smd rect (at 2.55 7.65) (size 1 1) (layers "F.Cu" "F.Mask") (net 32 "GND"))
  (pad "65" smd rect (at 5.95 4.25) (size 1 1) (layers "F.Cu" "F.Mask") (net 32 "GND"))
  (pad "66" smd rect (at 5.95 2.55) (size 1 1) (layers "F.Cu" "F.Mask") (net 32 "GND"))
  (pad "67" smd rect (at 5.95 0.85) (size 1 1) (layers "F.Cu" "F.Mask"))
  (pad "68" smd rect (at 5.95 -0.85) (size 1 1) (layers "F.Cu" "F.Mask"))
  (pad "69" smd rect (at 5.95 -2.55) (size 1 1) (layers "F.Cu" "F.Mask"))
  (pad "70" smd rect (at 5.95 -4.25) (size 1 1) (layers "F.Cu" "F.Mask"))
  (pad "71" smd rect (at 2.55 -7.65) (size 1 1) (layers "F.Cu" "F.Mask") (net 32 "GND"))
  (pad "72" smd rect (at 0.85 -7.65) (size 1 1) (layers "F.Cu" "F.Mask") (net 32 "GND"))
  (pad "73" smd rect (at -0.85 -7.65) (size 1 1) (layers "F.Cu" "F.Mask") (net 32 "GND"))
  (pad "74" smd rect (at -2.55 -7.65) (size 1 1) (layers "F.Cu" "F.Mask") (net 32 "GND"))
  (pad "75" smd rect (at -4.25 -4.25) (size 1 1) (layers "F.Cu" "F.Mask"))
  (pad "76" smd rect (at -4.25 -2.55) (size 1 1) (layers "F.Cu" "F.Mask"))
  (pad "77" smd rect (at -4.25 -0.85) (size 1 1) (layers "F.Cu" "F.Mask"))
  (pad "78" smd rect (at -4.25 0.85) (size 1 1) (layers "F.Cu" "F.Mask"))
  (pad "79" smd rect (at -4.25 2.55) (size 1 1) (layers "F.Cu" "F.Mask"))
  (pad "80" smd rect (at -4.25 4.25) (size 1 1) (layers "F.Cu" "F.Mask"))
  (pad "81" smd rect (at -2.55 5.95) (size 1 1) (layers "F.Cu" "F.Mask") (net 32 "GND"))
  (pad "82" smd rect (at -0.85 5.95) (size 1 1) (layers "F.Cu" "F.Mask") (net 32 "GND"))
  (pad "83" smd rect (at 0.85 5.95) (size 1 1) (layers "F.Cu" "F.Mask") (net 32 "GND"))
  (pad "84" smd rect (at 2.55 5.95) (size 1 1) (layers "F.Cu" "F.Mask"))
  (pad "85" smd rect (at 4.25 4.25) (size 1 1) (layers "F.Cu" "F.Mask"))
  (pad "86" smd rect (at 4.25 2.55) (size 1 1) (layers "F.Cu" "F.Mask"))
  (pad "87" smd rect (at 4.25 0.85) (size 1 1) (layers "F.Cu" "F.Mask"))
  (pad "88" smd rect (at 4.25 -0.85) (size 1 1) (layers "F.Cu" "F.Mask"))
  (pad "89" smd rect (at 4.25 -2.55) (size 1 1) (layers "F.Cu" "F.Mask"))
  (pad "90" smd rect (at 4.25 -4.25) (size 1 1) (layers "F.Cu" "F.Mask"))
  (pad "91" smd rect (at 2.55 -5.95) (size 1 1) (layers "F.Cu" "F.Mask"))
  (pad "92" smd rect (at 0.85 -5.95) (size 1 1) (layers "F.Cu" "F.Mask") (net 32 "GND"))
  (pad "93" smd rect (at -0.85 -5.95) (size 1 1) (layers "F.Cu" "F.Mask") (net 32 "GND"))
  (pad "94" smd rect (at -2.55 -5.95) (size 1 1) (layers "F.Cu" "F.Mask") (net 32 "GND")))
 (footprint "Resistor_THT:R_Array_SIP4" (layer "F.Cu") (at 149.88 139.5)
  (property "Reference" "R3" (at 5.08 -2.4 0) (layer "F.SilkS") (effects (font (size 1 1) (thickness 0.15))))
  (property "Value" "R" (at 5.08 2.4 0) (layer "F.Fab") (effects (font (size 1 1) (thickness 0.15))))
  (pad "1" thru_hole rect (at 0 0) (size 1.6 1.6) (drill 0.8) (layers "*.Cu" "*.Mask") (remove_unused_layers no) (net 32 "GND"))
  (pad "2" thru_hole oval (at 2.54 0) (size 1.6 1.6) (drill 0.8) (layers "*.Cu" "*.Mask") (remove_unused_layers no) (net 10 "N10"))
  (pad "3" thru_hole oval (at 5.08 0) (size 1.6 1.6) (drill 0.8) (layers "*.Cu" "*.Mask") (remove_unused_layers no))
  (pad "4" thru_hole oval (at 7.62 0) (size 1.6 1.6) (drill 0.8) (layers "*.Cu" "*.Mask") (remove_unused_layers no)))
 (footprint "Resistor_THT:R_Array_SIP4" (layer "F.Cu") (at 148.42 128)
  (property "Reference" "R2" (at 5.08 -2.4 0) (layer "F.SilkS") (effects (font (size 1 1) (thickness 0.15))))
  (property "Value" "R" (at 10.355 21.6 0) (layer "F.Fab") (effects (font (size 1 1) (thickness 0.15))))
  (pad "1" thru_hole rect (at 0 0) (size 1.6 1.6) (drill 0.8) (layers "*.Cu" "*.Mask") (remove_unused_layers no) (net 39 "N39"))
  (pad "2" thru_hole oval (at 2.54 0) (size 1.6 1.6) (drill 0.8) (layers "*.Cu" "*.Mask") (remove_unused_layers no) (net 11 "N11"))
  (pad "3" thru_hole oval (at 5.08 0) (size 1.6 1.6) (drill 0.8) (layers "*.Cu" "*.Mask") (remove_unused_layers no))
  (pad "4" thru_hole oval (at 7.62 0) (size 1.6 1.6) (drill 0.8) (layers "*.Cu" "*.Mask") (remove_unused_layers no)))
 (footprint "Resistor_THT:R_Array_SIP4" (layer "F.Cu") (at 145.675 117.5)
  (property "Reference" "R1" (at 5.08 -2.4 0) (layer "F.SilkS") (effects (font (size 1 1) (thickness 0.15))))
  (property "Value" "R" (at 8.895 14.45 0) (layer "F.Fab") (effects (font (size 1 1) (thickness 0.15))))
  (pad "1" thru_hole rect (at 0 0) (size 1.6 1.6) (drill 0.8) (layers "*.Cu" "*.Mask") (remove_unused_layers no) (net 39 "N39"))
  (pad "2" thru_hole oval (at 2.54 0) (size 1.6 1.6) (drill 0.8) (layers "*.Cu" "*.Mask") (remove_unused_layers no) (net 32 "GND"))
  (pad "3" thru_hole oval (at 5.08 0) (size 1.6 1.6) (drill 0.8) (layers "*.Cu" "*.Mask") (remove_unused_layers no))
  (pad "4" thru_hole oval (at 7.62 0) (size 1.6 1.6) (drill 0.8) (layers "*.Cu" "*.Mask") (remove_unused_layers no)))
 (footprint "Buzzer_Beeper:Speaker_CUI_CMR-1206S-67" (layer "F.Cu") (at 133 138)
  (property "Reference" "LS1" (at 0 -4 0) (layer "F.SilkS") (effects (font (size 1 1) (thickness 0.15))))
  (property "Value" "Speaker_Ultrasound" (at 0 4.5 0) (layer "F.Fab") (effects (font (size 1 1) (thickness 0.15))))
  (pad "1" smd rect (at -5.4 2.3 180) (size 1.5 2) (layers "F.Cu" "F.Mask") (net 27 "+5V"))
  (pad "2" smd rect (at 5.4 2.3 180) (size 1.5 2) (layers "F.Cu" "F.Mask") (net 6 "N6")))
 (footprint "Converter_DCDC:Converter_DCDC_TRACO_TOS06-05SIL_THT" (layer "F.Cu") (at 191 71.68)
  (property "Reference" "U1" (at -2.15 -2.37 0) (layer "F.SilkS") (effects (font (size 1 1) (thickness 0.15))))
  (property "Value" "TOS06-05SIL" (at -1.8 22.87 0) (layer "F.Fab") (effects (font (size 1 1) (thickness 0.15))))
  (pad "1" thru_hole rect (at 0 0) (size 2.1 2.1) (drill 1.3) (layers "*.Cu" "*.Mask") (remove_unused_layers no) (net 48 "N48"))
  (pad "2" thru_hole circle (at 0 2.54) (size 2.1 2.1) (drill 1.3) (layers "*.Cu" "*.Mask") (remove_unused_layers no) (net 32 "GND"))
  (pad "3" thru_hole circle (at 0 5.08) (size 2.1 2.1) (drill 1.3) (layers "*.Cu" "*.Mask") (remove_unused_layers no) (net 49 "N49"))
  (pad "4" thru_hole circle (at 0 17.78) (size 2.1 2.1) (drill 1.3) (layers "*.Cu" "*.Mask") (remove_unused_layers no) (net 27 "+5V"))
  (pad "5" thru_hole circle (at 0 20.32) (size 2.1 2.1) (drill 1.3) (layers "*.Cu" "*.Mask") (remove_unused_layers no) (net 32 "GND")))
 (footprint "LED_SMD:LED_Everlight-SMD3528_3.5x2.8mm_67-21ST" (layer "F.Cu") (at 175.19 117)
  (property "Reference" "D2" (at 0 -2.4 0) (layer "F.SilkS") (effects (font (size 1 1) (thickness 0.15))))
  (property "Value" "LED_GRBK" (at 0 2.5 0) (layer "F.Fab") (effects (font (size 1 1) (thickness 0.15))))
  (pad "1" smd roundrect (at -1.34 0) (size 1.1 2.1) (layers "F.Cu" "F.Mask" "F.Paste") (roundrect_rratio 0.15) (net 32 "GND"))
  (pad "2" smd roundrect (at 0.81 0) (size 2.1 2.1) (layers "F.Cu" "F.Mask" "F.Paste") (roundrect_rratio 0.15) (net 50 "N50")))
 (gr_rect (start 75 52) (end 227.5 160.5) (stroke (width 0.05) (type default)) (fill no) (layer "Edge.Cuts"))
 (segment (start 138.5 143.5) (end 138.4 143.4) (width 0.2) (layer "F.Cu") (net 6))
 (segment (start 133 148.5) (end 138 143.5) (width 0.2) (layer "F.Cu") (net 6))
 (segment (start 85 97.5) (end 85 131) (width 0.2) (layer "F.Cu") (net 6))
 (segment (start 85 131) (end 102.5 148.5) (width 0.2) (layer "F.Cu") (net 6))
 (segment (start 138.4 143.4) (end 138.4 140.3) (width 0.2) (layer "F.Cu") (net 6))
 (segment (start 138 143.5) (end 138.5 143.5) (width 0.2) (layer "F.Cu") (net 6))
 (segment (start 90.76 93.64) (end 88.86 93.64) (width 0.2) (layer "F.Cu") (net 6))
 (segment (start 88.86 93.64) (end 85 97.5) (width 0.2) (layer "F.Cu") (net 6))
 (segment (start 102.5 148.5) (end 133 148.5) (width 0.2) (layer "F.Cu") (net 6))
 (segment (start 128.199 105.239) (end 150.96 128) (width 0.2) (layer "F.Cu") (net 11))
 (segment (start 90.76 106.34) (end 91.861 105.239) (width 0.2) (layer "F.Cu") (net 11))
 (segment (start 91.861 105.239) (end 128.199 105.239) (width 0.2) (layer "F.Cu") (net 11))
 (segment (start 150.854 102.854) (end 150.854 100.751) (width 0.2) (layer "F.Cu") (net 13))
 (segment (start 151.155 100.45) (end 152.355 100.45) (width 0.2) (layer "F.Cu") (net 13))
 (segment (start 151 103) (end 150.854 102.854) (width 0.2) (layer "F.Cu") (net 13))
 (segment (start 150.854 100.751) (end 151.155 100.45) (width 0.2) (layer "F.Cu") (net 13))
 (via (at 151 103) (size 0.6) (drill 0.3) (layers "F.Cu" "B.Cu") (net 13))
 (segment (start 149 102.361) (end 150.361 102.361) (width 0.2) (layer "B.Cu") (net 13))
 (segment (start 90.76 111.42) (end 89.659 110.319) (width 0.2) (layer "B.Cu") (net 13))
 (segment (start 150.361 102.361) (end 151 103) (width 0.2) (layer "B.Cu") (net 13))
 (segment (start 90.64195 102.361) (end 149 102.361) (width 0.2) (layer "B.Cu") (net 13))
 (segment (start 89.659 110.319) (end 89.659 103.34395) (width 0.2) (layer "B.Cu") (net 13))
 (segment (start 89.659 103.34395) (end 90.64195 102.361) (width 0.2) (layer "B.Cu") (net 13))
 (segment (start 174.635 124.365) (end 174.635 120.4) (width 0.2) (layer "F.Cu") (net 27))
 (segment (start 165 134) (end 174.635 124.365) (width 0.2) (layer "F.Cu") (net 27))
 (segment (start 183 120.5) (end 182.9 120.4) (width 0.2) (layer "F.Cu") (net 27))
 (segment (start 134 132) (end 132 134) (width 0.2) (layer "F.Cu") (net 27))
 (segment (start 132 134) (end 165 134) (width 0.2) (layer "F.Cu") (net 27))
 (segment (start 183.5 120.5) (end 183 120.5) (width 0.2) (layer "F.Cu") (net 27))
 (segment (start 182.9 120.4) (end 174.635 120.4) (width 0.2) (layer "F.Cu") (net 27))
 (segment (start 127.6 138.4) (end 132 134) (width 0.2) (layer "F.Cu") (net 27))
 (segment (start 191 89.46) (end 194.46 89.46) (width 0.2) (layer "F.Cu") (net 27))
 (segment (start 197.5 92.5) (end 197.5 106.5) (width 0.2) (layer "F.Cu") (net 27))
 (segment (start 197.5 106.5) (end 183.5 120.5) (width 0.2) (layer "F.Cu") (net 27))
 (segment (start 194.46 89.46) (end 197.5 92.5) (width 0.2) (layer "F.Cu") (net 27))
 (segment (start 136.5 132) (end 134 132) (width 0.2) (layer "F.Cu") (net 27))
 (segment (start 127.6 140.3) (end 127.6 138.4) (width 0.2) (layer "F.Cu") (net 27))
 (via (at 136.5 132) (size 0.6) (drill 0.3) (layers "F.Cu" "B.Cu") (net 27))
 (segment (start 106 88.56) (end 142.6942 88.56) (width 0.2) (layer "B.Cu") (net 27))
 (segment (start 146.776 116.399) (end 146.776 121.1511) (width 0.2) (layer "B.Cu") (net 27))
 (segment (start 146.776 121.724) (end 136.5 132) (width 0.2) (layer "B.Cu") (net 27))
 (segment (start 153.302 99.1678) (end 153.302 109.873) (width 0.2) (layer "B.Cu") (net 27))
 (segment (start 153.302 109.873) (end 146.776 116.399) (width 0.2) (layer "B.Cu") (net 27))
 (segment (start 146.776 121.1511) (end 146.776 121.724) (width 0.2) (layer "B.Cu") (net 27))
 (segment (start 142.6942 88.56) (end 153.302 99.1678) (width 0.2) (layer "B.Cu") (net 27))
 (segment (start 127.561 140.601) (end 90.76 103.8) (width 0.2) (layer "B.Cu") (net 10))
 (segment (start 152.42 139.5) (end 151.319 140.601) (width 0.2) (layer "B.Cu") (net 10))
 (segment (start 151.319 140.601) (end 127.561 140.601) (width 0.2) (layer "B.Cu") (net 10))
 (segment (start 172.999 114.394) (end 172.999 120.164) (width 0.2) (layer "F.Cu") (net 31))
 (segment (start 172.999 120.164) (end 173.235 120.4) (width 0.2) (layer "F.Cu") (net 31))
 (segment (start 153.555 94.95) (end 172.999 114.394) (width 0.2) (layer "F.Cu") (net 31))
 (segment (start 152.355 94.95) (end 153.555 94.95) (width 0.2) (layer "F.Cu") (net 31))
 (segment (start 136.506 82.901) (end 136.205 82.6) (width 0.2) (layer "F.Cu") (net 32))
 (segment (start 141.705 99) (end 143.405 99) (width 0.2) (layer "F.Cu") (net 32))
 (segment (start 173.85 117) (end 173.85 120.776968) (width 0.2) (layer "F.Cu") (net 32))
 (segment (start 140.005 85.4) (end 141.705 85.4) (width 0.2) (layer "F.Cu") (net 32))
 (segment (start 189.5 75.72) (end 189.5 90.5) (width 0.2) (layer "F.Cu") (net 32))
 (segment (start 136.205 82.6) (end 136.205 81.4) (width 0.2) (layer "F.Cu") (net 32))
 (segment (start 137.504 89.699) (end 137.406 89.797) (width 0.2) (layer "F.Cu") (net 32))
 (segment (start 147.155 84.45) (end 152.355 84.45) (width 0.2) (layer "F.Cu") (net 32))
 (segment (start 145.105 100.7) (end 142.429 103.376) (width 0.2) (layer "F.Cu") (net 32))
 (segment (start 138.405 82.6) (end 138.104 82.901) (width 0.2) (layer "F.Cu") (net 32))
 (segment (start 138.405 81.4) (end 138.405 82.6) (width 0.2) (layer "F.Cu") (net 32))
 (segment (start 137.406 89.797) (end 137.406 94.799) (width 0.2) (layer "F.Cu") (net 32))
 (segment (start 191 74.22) (end 189.5 75.72) (width 0.2) (layer "F.Cu") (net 32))
 (segment (start 146.055 84.45) (end 152.355 84.45) (width 0.2) (layer "F.Cu") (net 32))
 (segment (start 148.505 97.3) (end 148.505 95.6) (width 0.2) (layer "F.Cu") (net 32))
 (segment (start 140.005 99) (end 141.705 99) (width 0.2) (layer "F.Cu") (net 32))
 (segment (start 133.55104 85.55) (end 132.755 85.55) (width 0.2) (layer "F.Cu") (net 32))
 (segment (start 141.705 85.4) (end 141.705 87.1) (width 0.2) (layer "F.Cu") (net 32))
 (segment (start 140.005 87.1) (end 140.005 88.702) (width 0.2) (layer "F.Cu") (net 32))
 (segment (start 139.505 81.4) (end 138.405 81.4) (width 0.2) (layer "F.Cu") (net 32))
 (segment (start 138.104 82.901) (end 136.506 82.901) (width 0.2) (layer "F.Cu") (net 32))
 (segment (start 136.605 97.3) (end 138.305 99) (width 0.2) (layer "F.Cu") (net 32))
 (segment (start 189.5 90.5) (end 191 92) (width 0.2) (layer "F.Cu") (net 32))
 (segment (start 138.305 99) (end 140.005 99) (width 0.2) (layer "F.Cu") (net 32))
 (segment (start 136.205 82.89604) (end 133.55104 85.55) (width 0.2) (layer "F.Cu") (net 32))
 (segment (start 141.705 100.7) (end 140.005 100.7) (width 0.2) (layer "F.Cu") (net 32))
 (segment (start 143.405 99) (end 143.405 100.7) (width 0.2) (layer "F.Cu") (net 32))
 (segment (start 145.105 85.4) (end 143.405 85.4) (width 0.2) (layer "F.Cu") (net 32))
 (segment (start 191 92) (end 173.85 109.15) (width 0.2) (layer "F.Cu") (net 32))
 (segment (start 143.405 87.1) (end 141.705 87.1) (width 0.2) (layer "F.Cu") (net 32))
 (segment (start 173.85 120.776968) (end 173.575968 121.051) (width 0.2) (layer "F.Cu") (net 32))
 (segment (start 139.505 84.9) (end 139.505 81.4) (width 0.2) (layer "F.Cu") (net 32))
 (segment (start 145.305 81.4) (end 145.305 82.6) (width 0.2) (layer "F.Cu") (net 32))
 (segment (start 142.429 111.714) (end 148.215 117.5) (width 0.2) (layer "F.Cu") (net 32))
 (segment (start 140.005 100.7) (end 140.005 99) (width 0.2) (layer "F.Cu") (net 32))
 (segment (start 143.405 100.7) (end 145.105 100.7) (width 0.2) (layer "F.Cu") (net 32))
 (segment (start 145.105 85.4) (end 146.055 84.45) (width 0.2) (layer "F.Cu") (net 32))
 (segment (start 136.205 81.4) (end 136.205 82.89604) (width 0.2) (layer "F.Cu") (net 32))
 (segment (start 140.005 85.4) (end 139.505 84.9) (width 0.2) (layer "F.Cu") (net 32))
 (segment (start 137.406 94.799) (end 136.605 95.6) (width 0.2) (layer "F.Cu") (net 32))
 (segment (start 141.705 99) (end 141.705 100.7) (width 0.2) (layer "F.Cu") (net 32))
 (segment (start 145.105 100.7) (end 148.505 97.3) (width 0.2) (layer "F.Cu") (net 32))
 (segment (start 139.008 89.699) (end 137.504 89.699) (width 0.2) (layer "F.Cu") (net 32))
 (segment (start 145.305 82.6) (end 147.155 84.45) (width 0.2) (layer "F.Cu") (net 32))
 (segment (start 140.005 88.702) (end 139.008 89.699) (width 0.2) (layer "F.Cu") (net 32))
 (segment (start 143.405 85.4) (end 143.405 87.1) (width 0.2) (layer "F.Cu") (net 32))
 (segment (start 142.429 103.376) (end 142.429 111.714) (width 0.2) (layer "F.Cu") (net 32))
 (segment (start 151.766 121.051) (end 148.215 117.5) (width 0.2) (layer "F.Cu") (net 32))
 (segment (start 140.005 87.1) (end 140.005 85.4) (width 0.2) (layer "F.Cu") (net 32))
 (segment (start 173.85 109.15) (end 173.85 117) (width 0.2) (layer "F.Cu") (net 32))
 (segment (start 136.605 95.6) (end 136.605 97.3) (width 0.2) (layer "F.Cu") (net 32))
 (segment (start 173.575968 121.051) (end 151.766 121.051) (width 0.2) (layer "F.Cu") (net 32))
 (segment (start 147.319 136.939) (end 149.88 139.5) (width 0.2) (layer "B.Cu") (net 32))
 (segment (start 147.319 118.396) (end 147.319 136.939) (width 0.2) (layer "B.Cu") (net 32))
 (segment (start 148.215 117.5) (end 147.319 118.396) (width 0.2) (layer "B.Cu") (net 32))
 (segment (start 150 100.90896) (end 151.55896 99.35) (width 0.2) (layer "F.Cu") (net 39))
 (segment (start 151.55896 99.35) (end 152.355 99.35) (width 0.2) (layer "F.Cu") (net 39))
 (segment (start 152.399 124.224) (end 145.675 117.5) (width 0.2) (layer "F.Cu") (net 39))
 (segment (start 152.399 128.45605) (end 152.399 124.224) (width 0.2) (layer "F.Cu") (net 39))
 (segment (start 151.75405 129.101) (end 152.399 128.45605) (width 0.2) (layer "F.Cu") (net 39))
 (segment (start 149.521 129.101) (end 151.75405 129.101) (width 0.2) (layer "F.Cu") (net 39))
 (segment (start 148.42 128) (end 149.521 129.101) (width 0.2) (layer "F.Cu") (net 39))
 (segment (start 150 106.5) (end 150 100.90896) (width 0.2) (layer "F.Cu") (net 39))
 (via (at 150 106.5) (size 0.6) (drill 0.3) (layers "F.Cu" "B.Cu") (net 39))
 (segment (start 145.675 117.5) (end 145.675 110.825) (width 0.2) (layer "B.Cu") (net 39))
 (segment (start 145.675 110.825) (end 150 106.5) (width 0.2) (layer "B.Cu") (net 39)))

